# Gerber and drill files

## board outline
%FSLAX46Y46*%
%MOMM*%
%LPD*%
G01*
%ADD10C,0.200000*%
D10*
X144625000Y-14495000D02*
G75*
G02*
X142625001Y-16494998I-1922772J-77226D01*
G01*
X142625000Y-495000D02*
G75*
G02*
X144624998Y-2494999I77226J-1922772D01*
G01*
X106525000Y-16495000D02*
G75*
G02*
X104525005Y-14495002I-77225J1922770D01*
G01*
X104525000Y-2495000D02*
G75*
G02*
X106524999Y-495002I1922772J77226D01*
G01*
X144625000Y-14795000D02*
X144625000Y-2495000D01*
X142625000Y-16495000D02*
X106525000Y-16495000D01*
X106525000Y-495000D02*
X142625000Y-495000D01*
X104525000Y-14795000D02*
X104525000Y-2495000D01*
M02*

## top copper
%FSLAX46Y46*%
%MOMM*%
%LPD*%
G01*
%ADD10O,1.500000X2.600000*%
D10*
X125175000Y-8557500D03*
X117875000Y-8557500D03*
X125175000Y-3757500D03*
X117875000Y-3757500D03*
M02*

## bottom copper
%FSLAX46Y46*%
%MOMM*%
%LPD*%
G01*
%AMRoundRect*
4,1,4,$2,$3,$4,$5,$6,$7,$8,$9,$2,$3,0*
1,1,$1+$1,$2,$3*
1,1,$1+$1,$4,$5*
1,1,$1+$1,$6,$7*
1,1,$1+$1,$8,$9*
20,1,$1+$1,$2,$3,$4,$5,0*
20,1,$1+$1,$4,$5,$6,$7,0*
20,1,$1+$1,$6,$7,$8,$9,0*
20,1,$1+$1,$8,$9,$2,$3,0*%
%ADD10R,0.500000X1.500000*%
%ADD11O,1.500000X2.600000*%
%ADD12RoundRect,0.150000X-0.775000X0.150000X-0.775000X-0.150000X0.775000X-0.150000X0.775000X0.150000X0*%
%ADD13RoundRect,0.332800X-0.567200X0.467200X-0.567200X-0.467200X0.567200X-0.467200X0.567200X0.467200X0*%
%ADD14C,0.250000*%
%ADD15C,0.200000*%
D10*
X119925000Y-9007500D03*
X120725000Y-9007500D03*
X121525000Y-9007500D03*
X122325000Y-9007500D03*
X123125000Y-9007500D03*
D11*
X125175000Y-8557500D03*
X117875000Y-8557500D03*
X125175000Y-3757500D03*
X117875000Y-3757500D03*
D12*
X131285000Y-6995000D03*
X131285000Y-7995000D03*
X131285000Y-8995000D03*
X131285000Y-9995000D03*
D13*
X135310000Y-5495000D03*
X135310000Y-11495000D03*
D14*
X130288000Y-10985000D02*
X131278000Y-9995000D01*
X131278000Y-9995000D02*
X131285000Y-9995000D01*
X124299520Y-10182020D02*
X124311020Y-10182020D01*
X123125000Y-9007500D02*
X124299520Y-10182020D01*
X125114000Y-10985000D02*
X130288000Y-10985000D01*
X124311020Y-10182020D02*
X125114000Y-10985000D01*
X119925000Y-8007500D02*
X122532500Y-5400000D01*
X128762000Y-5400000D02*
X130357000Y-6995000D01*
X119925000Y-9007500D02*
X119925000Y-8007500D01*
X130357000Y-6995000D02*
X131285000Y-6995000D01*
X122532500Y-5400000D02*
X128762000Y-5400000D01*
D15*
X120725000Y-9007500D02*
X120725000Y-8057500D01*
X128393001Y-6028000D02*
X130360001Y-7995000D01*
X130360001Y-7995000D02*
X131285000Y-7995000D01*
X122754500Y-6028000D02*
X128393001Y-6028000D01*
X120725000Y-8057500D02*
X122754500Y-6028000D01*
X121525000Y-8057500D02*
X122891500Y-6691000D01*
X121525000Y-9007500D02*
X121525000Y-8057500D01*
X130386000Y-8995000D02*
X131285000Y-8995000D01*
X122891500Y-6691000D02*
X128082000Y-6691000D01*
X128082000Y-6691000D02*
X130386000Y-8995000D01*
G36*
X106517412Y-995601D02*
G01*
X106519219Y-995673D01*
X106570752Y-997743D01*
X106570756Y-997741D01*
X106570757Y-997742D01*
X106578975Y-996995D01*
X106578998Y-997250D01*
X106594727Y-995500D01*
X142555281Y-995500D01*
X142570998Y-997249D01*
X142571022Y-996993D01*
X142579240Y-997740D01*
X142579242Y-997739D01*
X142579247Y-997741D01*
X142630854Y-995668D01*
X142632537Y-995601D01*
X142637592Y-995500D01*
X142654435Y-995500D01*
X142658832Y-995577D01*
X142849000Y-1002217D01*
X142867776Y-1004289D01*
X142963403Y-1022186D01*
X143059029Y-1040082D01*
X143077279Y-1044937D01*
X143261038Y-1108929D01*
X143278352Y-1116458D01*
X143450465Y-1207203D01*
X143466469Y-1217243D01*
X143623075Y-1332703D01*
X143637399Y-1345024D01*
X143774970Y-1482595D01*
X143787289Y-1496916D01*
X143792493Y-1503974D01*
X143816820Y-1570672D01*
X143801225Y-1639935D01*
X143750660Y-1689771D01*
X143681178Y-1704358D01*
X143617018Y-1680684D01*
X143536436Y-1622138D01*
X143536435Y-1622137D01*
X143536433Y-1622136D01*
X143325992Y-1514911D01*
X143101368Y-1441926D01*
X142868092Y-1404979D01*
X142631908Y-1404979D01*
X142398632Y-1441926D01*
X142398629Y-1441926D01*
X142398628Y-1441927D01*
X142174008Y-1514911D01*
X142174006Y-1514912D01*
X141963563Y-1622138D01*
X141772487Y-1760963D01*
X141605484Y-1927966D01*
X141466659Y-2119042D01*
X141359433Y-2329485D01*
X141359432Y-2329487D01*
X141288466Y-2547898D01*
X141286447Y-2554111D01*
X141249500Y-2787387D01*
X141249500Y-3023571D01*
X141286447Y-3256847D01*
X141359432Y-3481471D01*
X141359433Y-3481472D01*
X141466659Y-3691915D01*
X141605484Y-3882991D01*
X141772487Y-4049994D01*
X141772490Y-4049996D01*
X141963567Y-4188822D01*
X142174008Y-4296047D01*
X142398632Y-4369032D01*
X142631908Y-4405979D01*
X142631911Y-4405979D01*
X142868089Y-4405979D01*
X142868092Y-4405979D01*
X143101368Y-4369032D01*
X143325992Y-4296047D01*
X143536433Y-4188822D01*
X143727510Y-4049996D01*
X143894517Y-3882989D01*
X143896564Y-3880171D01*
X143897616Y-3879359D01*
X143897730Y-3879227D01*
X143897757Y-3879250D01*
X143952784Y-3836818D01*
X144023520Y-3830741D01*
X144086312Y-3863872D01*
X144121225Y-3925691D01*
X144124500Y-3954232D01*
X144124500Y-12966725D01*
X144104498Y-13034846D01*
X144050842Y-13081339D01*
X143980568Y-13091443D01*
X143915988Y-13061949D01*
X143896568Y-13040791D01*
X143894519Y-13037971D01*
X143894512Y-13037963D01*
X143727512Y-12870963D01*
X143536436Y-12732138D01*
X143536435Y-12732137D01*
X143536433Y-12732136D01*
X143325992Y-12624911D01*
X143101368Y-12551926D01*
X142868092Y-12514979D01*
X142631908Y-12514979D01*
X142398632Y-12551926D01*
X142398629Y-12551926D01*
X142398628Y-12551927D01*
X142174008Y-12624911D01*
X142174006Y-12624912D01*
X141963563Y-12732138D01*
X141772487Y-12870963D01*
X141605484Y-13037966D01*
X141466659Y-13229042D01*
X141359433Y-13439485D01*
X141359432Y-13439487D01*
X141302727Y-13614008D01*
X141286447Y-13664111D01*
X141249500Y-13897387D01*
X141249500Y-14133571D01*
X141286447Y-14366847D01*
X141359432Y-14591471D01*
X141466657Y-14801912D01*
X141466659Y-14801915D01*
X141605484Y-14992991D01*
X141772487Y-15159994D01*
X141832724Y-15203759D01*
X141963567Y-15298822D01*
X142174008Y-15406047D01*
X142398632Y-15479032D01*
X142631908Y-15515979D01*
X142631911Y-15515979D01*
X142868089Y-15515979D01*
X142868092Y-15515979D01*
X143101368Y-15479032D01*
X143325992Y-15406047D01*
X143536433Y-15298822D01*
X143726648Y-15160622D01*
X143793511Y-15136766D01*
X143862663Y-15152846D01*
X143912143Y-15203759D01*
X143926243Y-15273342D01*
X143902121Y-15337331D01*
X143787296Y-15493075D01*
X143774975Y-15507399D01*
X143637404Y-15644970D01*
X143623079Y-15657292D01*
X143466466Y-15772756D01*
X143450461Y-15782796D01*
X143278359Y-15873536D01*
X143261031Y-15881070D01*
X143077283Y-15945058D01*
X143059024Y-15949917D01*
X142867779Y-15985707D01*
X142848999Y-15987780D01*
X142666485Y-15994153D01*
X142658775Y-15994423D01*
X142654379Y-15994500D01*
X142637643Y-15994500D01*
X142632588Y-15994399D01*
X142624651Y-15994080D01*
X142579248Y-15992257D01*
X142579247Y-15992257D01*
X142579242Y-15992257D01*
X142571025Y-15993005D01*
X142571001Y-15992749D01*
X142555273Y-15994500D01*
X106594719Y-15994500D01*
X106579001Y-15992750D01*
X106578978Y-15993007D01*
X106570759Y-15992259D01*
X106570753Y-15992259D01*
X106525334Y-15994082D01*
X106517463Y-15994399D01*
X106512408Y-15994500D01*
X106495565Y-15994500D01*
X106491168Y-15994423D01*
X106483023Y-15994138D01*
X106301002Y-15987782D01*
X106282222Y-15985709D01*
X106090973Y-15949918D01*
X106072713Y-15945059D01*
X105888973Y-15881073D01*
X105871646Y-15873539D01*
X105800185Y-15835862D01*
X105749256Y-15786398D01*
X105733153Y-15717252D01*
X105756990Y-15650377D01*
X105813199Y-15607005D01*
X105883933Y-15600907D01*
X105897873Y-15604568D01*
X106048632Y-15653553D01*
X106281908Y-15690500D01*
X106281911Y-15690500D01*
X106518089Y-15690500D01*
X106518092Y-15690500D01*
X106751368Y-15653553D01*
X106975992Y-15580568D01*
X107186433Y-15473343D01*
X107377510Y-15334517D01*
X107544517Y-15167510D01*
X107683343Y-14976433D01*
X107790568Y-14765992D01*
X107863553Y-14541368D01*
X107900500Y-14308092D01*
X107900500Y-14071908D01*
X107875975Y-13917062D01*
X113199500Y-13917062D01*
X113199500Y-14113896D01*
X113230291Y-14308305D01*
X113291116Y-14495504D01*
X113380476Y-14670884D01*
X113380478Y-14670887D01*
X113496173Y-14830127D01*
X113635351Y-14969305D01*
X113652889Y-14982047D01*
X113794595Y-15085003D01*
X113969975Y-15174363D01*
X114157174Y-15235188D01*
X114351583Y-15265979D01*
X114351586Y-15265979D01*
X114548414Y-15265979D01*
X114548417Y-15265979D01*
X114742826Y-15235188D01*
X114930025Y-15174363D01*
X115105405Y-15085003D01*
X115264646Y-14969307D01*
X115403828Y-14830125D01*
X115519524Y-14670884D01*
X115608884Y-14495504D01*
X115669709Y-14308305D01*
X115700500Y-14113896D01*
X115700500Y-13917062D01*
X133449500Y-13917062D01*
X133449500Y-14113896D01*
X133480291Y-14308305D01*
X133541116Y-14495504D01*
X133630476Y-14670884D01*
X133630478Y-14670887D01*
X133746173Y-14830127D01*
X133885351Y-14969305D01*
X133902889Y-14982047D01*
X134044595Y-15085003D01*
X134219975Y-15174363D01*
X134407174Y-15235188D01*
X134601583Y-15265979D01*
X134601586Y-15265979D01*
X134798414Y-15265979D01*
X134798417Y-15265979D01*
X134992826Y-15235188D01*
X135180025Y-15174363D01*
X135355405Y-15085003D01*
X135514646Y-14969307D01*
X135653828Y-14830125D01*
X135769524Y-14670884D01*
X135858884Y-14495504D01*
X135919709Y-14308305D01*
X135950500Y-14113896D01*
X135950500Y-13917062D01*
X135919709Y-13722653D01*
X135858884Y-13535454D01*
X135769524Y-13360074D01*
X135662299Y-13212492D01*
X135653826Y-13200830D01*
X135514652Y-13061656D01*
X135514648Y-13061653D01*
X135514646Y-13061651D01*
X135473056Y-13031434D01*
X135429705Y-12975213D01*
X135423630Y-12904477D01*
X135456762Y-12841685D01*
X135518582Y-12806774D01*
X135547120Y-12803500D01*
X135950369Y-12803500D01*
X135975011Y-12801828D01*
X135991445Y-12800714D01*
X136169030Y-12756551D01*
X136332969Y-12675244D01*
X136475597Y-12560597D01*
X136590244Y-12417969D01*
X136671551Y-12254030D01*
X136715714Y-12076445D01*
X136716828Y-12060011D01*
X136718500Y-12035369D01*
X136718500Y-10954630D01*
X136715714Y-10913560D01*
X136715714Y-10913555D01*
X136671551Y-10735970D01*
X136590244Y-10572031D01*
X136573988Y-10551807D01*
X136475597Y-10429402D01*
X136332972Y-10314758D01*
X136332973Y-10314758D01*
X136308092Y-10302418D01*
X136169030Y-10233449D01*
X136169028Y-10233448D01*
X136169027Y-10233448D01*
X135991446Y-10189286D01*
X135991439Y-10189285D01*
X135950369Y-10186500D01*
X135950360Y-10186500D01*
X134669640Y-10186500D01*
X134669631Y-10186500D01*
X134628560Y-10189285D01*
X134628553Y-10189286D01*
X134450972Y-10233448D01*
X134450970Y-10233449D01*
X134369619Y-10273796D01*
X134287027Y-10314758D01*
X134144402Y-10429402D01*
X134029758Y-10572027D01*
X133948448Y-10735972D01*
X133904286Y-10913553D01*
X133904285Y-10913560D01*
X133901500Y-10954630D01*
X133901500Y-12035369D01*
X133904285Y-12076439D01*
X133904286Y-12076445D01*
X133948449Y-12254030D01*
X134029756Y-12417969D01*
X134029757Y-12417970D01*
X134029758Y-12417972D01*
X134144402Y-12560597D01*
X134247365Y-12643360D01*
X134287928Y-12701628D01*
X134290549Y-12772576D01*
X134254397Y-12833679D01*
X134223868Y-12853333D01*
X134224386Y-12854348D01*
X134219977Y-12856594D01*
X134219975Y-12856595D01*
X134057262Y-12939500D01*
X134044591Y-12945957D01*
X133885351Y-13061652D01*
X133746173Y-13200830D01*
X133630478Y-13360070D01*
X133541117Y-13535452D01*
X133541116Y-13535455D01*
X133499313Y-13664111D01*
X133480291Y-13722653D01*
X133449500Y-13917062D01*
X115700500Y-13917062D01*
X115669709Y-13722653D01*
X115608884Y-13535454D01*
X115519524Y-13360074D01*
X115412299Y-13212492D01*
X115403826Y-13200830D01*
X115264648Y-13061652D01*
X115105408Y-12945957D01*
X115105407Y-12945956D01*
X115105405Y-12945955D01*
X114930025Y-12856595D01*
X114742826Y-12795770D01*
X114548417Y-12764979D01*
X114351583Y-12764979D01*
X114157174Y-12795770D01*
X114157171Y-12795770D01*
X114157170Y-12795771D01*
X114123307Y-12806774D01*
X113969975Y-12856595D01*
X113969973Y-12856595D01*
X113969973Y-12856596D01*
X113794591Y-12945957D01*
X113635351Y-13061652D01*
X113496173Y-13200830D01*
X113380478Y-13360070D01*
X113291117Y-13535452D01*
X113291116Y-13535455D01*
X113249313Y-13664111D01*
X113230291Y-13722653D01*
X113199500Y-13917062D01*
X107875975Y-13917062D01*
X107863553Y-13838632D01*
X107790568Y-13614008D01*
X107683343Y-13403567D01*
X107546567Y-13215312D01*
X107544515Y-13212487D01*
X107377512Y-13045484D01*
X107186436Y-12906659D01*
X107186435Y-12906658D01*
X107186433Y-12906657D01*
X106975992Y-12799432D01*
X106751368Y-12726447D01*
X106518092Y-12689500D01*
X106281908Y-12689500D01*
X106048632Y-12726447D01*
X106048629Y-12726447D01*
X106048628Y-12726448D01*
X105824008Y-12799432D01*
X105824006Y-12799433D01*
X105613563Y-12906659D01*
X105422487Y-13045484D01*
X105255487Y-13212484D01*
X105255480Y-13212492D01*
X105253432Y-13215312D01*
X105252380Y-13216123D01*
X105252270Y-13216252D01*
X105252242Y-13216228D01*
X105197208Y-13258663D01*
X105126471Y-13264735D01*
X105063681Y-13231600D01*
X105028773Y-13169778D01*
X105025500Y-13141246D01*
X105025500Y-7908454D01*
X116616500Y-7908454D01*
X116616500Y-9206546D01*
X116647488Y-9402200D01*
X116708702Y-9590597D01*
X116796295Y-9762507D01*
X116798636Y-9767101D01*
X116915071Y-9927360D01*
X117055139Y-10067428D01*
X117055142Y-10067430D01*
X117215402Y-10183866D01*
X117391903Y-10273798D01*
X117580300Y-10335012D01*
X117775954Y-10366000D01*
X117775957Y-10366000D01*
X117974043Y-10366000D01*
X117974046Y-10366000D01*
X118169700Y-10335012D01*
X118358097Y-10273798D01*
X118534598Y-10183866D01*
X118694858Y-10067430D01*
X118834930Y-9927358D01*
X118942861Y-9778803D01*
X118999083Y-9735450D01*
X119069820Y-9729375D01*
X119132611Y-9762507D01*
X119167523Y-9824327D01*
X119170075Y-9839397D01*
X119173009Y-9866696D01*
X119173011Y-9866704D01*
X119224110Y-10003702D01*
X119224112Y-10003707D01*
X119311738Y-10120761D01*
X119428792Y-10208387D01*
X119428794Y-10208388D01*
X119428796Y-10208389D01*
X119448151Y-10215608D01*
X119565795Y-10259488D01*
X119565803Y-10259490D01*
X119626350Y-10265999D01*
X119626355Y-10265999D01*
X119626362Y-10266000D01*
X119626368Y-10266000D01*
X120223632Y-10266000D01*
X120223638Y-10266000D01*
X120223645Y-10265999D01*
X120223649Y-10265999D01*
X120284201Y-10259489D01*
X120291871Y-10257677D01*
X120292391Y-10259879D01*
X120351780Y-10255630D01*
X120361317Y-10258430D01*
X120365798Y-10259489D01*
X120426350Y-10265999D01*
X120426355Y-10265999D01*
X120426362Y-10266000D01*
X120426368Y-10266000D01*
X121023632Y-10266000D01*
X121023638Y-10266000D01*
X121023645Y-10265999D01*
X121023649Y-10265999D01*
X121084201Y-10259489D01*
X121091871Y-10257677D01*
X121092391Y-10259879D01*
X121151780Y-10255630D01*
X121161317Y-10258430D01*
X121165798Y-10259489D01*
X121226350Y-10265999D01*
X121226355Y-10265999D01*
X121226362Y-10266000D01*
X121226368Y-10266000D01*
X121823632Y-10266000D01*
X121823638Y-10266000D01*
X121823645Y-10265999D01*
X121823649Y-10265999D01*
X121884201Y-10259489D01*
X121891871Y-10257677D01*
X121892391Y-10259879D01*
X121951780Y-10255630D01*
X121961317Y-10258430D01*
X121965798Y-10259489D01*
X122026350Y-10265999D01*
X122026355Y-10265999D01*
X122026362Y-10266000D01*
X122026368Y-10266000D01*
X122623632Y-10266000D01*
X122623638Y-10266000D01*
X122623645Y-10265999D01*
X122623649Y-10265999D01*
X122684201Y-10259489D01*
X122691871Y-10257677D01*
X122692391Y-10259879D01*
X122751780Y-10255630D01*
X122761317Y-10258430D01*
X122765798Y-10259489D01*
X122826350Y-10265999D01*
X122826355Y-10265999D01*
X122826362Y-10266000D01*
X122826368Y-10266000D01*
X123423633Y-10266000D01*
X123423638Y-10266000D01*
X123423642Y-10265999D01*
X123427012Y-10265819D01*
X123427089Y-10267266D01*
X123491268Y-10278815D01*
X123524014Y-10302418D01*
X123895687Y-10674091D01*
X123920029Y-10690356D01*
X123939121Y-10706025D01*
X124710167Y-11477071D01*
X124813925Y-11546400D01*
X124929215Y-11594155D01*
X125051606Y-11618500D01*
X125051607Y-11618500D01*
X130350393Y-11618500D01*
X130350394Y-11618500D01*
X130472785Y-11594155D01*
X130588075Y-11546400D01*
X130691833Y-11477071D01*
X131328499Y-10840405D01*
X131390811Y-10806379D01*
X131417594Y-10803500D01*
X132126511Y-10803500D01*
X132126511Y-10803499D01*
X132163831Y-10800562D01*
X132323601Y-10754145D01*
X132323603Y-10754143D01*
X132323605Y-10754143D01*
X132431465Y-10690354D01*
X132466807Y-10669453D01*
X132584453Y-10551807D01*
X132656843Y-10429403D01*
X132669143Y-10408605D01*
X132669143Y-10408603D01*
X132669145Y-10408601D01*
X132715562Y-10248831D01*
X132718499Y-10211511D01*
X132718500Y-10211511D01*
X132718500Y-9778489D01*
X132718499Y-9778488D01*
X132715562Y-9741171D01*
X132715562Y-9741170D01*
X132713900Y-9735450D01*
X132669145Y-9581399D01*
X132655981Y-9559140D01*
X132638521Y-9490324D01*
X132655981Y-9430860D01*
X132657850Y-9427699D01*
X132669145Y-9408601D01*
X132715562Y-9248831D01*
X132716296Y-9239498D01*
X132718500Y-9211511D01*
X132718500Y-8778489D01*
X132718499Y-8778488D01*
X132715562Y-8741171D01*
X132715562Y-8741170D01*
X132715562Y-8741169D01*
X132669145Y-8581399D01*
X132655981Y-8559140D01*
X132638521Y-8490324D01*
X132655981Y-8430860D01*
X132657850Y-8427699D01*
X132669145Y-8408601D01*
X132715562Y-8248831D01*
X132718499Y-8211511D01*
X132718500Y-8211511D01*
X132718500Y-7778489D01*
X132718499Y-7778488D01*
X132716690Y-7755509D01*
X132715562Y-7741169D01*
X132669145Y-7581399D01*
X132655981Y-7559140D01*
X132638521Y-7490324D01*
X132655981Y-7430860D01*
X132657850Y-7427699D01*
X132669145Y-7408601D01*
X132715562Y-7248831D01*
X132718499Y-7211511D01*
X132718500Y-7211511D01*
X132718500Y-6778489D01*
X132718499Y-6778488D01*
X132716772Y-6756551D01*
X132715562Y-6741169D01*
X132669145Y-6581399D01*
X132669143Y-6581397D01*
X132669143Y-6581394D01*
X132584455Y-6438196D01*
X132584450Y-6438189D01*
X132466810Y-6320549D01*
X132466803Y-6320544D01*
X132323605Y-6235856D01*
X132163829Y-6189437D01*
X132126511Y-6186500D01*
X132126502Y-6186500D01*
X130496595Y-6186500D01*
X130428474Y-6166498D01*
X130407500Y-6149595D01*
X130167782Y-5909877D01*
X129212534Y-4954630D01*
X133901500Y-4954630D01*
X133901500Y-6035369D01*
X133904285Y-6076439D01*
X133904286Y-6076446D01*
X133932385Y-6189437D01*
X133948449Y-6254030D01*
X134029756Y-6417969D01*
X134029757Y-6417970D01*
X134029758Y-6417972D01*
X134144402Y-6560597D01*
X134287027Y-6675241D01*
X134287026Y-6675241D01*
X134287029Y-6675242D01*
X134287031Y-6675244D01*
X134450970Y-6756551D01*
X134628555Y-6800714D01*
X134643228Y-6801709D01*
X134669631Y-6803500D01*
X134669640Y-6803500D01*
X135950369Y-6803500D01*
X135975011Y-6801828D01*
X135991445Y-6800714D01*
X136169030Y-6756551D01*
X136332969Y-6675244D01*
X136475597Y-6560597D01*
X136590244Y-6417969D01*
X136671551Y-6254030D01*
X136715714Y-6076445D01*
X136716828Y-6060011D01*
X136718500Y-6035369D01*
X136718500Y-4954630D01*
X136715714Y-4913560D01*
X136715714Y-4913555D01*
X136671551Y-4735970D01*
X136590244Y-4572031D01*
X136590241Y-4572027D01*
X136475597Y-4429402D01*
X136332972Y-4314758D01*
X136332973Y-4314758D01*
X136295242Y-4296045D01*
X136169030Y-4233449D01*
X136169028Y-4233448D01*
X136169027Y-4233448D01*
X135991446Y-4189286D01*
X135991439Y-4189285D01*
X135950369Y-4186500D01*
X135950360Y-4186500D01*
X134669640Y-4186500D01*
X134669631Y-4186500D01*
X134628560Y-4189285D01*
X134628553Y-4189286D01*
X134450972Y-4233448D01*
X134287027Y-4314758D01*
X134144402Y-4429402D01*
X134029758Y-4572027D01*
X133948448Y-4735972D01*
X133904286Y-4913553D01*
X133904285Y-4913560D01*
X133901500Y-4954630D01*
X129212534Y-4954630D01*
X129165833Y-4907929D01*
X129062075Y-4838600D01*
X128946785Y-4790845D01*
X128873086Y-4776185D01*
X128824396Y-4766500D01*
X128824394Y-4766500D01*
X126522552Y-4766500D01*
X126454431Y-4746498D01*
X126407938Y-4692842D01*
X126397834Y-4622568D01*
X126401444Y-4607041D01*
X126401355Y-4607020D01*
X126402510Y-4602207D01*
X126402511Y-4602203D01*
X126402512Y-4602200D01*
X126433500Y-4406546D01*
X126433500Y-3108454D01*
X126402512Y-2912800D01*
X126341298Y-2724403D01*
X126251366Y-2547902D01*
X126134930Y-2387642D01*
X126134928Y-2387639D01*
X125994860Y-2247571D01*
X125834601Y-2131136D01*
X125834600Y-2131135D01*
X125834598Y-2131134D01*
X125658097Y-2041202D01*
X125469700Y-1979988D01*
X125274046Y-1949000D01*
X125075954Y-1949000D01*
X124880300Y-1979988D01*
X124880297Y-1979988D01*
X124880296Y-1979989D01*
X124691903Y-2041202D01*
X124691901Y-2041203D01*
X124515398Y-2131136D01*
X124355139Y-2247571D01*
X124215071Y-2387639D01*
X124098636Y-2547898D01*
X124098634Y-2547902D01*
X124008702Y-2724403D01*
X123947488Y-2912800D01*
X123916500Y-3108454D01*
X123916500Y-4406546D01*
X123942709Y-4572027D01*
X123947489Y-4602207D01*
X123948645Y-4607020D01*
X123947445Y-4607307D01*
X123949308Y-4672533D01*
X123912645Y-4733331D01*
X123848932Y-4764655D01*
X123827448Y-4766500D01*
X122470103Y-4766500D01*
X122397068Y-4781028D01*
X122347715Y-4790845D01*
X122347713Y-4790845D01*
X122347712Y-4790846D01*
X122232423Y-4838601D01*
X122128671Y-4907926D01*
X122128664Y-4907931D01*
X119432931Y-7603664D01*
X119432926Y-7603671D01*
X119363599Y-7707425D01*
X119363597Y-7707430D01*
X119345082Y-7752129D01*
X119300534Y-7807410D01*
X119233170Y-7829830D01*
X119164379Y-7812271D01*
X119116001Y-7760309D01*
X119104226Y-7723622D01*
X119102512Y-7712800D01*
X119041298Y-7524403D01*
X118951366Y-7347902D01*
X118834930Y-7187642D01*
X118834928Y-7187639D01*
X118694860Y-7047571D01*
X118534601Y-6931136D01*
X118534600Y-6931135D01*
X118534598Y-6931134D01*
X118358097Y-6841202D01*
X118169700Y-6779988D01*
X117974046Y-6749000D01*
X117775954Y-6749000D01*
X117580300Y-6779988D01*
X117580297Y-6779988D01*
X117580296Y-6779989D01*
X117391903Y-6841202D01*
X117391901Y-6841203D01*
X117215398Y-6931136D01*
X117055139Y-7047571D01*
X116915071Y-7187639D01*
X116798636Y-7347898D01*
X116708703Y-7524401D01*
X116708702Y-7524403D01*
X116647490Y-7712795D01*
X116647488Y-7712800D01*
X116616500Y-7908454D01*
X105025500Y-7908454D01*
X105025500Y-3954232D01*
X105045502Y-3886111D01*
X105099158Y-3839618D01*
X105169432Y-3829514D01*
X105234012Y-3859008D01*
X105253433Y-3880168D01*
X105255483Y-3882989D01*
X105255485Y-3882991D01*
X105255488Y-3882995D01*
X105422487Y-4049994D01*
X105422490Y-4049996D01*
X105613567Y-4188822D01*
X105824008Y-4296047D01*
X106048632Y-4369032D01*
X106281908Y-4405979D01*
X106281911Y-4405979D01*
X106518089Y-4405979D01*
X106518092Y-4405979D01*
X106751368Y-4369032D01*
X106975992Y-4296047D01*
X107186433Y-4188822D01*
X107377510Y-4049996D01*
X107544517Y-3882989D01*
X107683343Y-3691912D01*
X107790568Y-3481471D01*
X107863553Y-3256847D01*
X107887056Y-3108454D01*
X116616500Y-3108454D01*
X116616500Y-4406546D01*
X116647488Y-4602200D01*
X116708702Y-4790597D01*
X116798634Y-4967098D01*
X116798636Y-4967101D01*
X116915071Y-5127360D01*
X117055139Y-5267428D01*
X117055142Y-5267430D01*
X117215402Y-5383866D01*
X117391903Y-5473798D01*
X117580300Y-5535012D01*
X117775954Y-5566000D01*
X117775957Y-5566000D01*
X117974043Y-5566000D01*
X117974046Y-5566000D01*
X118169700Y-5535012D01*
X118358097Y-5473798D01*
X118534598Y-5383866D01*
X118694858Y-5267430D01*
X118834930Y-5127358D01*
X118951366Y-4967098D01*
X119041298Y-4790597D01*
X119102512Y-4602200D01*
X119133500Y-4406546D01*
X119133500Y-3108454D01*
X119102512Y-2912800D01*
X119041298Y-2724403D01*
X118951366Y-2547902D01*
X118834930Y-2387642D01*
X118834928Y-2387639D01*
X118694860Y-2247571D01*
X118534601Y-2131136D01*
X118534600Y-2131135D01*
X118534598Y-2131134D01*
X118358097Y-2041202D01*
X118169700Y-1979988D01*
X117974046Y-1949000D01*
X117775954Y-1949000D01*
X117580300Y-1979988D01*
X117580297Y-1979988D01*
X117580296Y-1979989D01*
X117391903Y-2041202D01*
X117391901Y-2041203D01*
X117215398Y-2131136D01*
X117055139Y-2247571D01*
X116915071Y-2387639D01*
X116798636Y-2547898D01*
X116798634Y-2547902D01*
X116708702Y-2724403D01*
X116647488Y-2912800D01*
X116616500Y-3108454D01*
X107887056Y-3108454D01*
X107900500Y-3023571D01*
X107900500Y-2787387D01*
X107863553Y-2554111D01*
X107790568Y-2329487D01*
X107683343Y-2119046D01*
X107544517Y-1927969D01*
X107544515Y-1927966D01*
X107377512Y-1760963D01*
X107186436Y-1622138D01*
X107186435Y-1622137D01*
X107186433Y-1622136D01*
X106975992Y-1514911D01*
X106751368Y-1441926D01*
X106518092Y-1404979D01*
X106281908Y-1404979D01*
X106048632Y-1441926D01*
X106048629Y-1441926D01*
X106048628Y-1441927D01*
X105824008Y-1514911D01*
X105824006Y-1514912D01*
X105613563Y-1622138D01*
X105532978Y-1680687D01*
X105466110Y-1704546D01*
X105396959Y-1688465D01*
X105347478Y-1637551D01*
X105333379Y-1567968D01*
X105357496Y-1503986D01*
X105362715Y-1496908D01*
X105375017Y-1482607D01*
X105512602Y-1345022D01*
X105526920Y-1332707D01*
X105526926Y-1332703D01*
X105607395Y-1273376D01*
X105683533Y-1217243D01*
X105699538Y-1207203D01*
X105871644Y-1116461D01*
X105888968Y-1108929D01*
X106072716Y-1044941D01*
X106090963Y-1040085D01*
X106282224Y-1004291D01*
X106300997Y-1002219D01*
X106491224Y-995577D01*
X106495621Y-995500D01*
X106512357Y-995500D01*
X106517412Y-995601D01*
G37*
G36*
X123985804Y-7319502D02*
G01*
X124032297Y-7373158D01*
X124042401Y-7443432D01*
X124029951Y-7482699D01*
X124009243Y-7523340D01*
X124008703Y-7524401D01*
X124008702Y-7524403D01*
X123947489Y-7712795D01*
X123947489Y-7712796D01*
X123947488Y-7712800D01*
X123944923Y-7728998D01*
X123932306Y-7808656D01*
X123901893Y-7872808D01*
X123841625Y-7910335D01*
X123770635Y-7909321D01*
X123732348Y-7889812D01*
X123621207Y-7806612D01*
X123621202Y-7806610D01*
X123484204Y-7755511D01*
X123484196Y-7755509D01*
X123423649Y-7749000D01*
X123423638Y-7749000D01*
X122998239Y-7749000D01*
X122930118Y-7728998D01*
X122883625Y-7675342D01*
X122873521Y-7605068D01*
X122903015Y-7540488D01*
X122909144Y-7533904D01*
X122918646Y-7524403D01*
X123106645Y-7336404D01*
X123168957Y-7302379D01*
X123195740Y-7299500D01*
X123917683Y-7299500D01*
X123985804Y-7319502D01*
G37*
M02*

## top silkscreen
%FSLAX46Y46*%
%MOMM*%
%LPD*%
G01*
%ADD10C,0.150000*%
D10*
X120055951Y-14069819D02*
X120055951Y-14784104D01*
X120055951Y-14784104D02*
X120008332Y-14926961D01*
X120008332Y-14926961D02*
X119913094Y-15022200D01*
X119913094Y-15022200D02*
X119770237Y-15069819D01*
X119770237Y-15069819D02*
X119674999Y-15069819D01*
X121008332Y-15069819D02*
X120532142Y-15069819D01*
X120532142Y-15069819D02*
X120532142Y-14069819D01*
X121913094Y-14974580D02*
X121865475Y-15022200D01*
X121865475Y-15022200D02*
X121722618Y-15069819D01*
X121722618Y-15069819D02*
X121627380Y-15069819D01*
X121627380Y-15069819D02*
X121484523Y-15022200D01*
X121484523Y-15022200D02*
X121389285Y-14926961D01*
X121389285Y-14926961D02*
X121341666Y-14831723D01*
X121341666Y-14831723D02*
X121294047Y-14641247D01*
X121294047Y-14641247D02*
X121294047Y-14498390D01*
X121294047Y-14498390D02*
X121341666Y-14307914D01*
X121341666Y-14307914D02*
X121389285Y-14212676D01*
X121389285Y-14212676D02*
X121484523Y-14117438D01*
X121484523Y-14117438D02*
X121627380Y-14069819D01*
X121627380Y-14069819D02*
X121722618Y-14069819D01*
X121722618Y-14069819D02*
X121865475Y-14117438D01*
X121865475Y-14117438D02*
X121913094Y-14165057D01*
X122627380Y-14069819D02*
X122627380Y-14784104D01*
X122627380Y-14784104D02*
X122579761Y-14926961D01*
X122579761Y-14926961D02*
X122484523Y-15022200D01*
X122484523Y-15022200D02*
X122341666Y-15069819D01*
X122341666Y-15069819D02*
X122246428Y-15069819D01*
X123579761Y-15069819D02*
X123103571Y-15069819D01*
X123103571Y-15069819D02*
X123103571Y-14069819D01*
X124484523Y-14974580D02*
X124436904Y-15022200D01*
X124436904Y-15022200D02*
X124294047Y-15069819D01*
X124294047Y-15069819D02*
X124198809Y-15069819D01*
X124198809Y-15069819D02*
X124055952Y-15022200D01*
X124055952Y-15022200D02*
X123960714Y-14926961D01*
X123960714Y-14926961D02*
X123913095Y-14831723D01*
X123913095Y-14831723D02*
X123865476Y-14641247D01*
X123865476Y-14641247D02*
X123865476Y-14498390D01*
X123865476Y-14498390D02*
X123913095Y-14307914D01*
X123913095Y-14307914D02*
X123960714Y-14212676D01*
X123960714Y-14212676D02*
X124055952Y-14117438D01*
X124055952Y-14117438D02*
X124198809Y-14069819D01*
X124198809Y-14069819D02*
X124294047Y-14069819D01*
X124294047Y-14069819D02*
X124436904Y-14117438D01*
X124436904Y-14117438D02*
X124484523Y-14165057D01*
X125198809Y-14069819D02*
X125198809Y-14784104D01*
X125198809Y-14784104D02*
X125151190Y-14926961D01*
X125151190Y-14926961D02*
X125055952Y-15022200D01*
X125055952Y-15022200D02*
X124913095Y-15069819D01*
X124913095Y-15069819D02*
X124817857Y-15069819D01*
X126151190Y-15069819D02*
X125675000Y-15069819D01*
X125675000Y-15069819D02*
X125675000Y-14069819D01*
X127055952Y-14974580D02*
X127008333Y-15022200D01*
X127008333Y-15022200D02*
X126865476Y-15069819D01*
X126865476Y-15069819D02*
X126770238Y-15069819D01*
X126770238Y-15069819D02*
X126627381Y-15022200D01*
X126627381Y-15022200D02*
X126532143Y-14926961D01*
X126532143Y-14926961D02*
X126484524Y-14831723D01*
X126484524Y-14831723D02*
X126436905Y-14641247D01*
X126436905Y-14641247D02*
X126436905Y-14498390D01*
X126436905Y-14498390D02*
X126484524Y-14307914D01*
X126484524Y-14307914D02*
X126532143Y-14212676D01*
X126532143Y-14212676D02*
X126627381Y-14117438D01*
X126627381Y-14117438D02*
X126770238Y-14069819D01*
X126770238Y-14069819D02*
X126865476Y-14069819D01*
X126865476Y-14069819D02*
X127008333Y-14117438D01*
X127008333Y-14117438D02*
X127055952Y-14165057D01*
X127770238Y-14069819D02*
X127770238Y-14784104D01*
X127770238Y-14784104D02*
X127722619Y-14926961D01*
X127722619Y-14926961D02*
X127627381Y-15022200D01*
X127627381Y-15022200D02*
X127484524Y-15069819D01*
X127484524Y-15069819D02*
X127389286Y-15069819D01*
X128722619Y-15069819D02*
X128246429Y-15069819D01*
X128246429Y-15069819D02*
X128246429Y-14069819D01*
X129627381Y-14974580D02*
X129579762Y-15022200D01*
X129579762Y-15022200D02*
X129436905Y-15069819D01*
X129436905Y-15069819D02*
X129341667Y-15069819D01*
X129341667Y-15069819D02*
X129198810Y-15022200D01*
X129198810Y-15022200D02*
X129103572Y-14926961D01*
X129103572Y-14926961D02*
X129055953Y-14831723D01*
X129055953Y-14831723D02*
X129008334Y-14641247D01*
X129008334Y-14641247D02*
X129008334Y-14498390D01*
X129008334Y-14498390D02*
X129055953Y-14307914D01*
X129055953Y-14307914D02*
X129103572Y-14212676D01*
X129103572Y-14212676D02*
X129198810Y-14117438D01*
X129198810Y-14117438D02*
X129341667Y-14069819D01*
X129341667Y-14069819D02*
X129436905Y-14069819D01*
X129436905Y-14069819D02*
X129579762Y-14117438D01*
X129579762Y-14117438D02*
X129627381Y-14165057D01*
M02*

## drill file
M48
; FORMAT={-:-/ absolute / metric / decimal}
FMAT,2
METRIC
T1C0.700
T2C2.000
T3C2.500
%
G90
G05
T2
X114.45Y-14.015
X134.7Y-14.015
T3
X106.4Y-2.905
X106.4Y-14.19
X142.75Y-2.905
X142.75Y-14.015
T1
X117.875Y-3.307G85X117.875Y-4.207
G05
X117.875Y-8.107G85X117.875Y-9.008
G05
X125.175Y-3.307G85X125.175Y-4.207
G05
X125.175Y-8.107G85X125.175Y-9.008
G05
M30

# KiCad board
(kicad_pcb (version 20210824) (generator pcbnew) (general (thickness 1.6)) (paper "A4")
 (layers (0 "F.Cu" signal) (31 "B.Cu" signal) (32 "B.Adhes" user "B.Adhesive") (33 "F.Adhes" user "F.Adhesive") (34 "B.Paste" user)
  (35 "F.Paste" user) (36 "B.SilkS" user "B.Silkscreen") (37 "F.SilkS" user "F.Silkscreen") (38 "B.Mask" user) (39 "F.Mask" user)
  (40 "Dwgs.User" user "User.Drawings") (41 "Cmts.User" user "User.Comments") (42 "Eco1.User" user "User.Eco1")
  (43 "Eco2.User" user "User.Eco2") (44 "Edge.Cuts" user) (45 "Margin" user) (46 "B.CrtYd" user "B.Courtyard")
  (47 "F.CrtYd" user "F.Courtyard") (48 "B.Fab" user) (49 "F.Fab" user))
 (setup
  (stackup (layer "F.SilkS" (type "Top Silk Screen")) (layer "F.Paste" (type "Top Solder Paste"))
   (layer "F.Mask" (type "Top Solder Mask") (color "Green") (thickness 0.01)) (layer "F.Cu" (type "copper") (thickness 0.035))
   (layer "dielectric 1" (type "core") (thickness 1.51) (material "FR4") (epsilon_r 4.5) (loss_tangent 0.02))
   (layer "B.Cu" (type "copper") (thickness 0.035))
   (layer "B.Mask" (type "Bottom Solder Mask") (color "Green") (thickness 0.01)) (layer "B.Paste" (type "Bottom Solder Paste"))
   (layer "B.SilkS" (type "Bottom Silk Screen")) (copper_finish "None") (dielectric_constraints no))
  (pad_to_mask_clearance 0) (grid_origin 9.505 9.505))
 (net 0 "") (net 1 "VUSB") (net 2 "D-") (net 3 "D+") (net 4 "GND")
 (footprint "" (layer "F.Cu") (at 136.255 14.205)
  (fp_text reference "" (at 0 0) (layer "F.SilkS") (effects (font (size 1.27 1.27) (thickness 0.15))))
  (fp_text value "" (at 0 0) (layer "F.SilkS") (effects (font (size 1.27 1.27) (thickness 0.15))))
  (pad "" np_thru_hole circle (at -1.555 -0.189521) (size 2 2) (drill 2) (layers F&B.Cu *.Mask)))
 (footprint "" (layer "F.Cu") (at 94.555 1.535)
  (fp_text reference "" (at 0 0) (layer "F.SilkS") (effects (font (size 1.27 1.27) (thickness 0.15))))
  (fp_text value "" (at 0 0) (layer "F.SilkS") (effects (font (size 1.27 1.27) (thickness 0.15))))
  (pad "" np_thru_hole circle (at 11.845 1.370479) (size 2.5 2.5) (drill 2.5) (layers F&B.Cu *.Mask)))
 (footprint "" (layer "F.Cu") (at 147.015 3.065)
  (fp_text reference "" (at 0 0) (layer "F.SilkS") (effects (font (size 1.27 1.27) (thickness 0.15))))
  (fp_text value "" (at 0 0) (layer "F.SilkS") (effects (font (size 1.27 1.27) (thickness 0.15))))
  (pad "" np_thru_hole circle (at -4.265 -0.159521) (size 2.5 2.5) (drill 2.5) (layers F&B.Cu *.Mask)))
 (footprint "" (layer "F.Cu") (at 94.295 7.445633)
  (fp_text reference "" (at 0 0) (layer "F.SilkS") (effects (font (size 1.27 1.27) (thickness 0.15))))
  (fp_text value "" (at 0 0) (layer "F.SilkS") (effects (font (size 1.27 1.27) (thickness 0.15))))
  (pad "" np_thru_hole circle (at 12.105 6.744367) (size 2.5 2.5) (drill 2.5) (layers F&B.Cu *.Mask)))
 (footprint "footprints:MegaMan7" (layer "F.Cu") (at 109.650838 8.415023)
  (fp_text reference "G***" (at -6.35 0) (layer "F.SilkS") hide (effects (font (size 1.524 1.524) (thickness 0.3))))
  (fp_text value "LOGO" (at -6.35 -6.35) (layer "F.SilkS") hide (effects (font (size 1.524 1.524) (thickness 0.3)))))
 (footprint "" (layer "F.Cu") (at 112.225 13.965)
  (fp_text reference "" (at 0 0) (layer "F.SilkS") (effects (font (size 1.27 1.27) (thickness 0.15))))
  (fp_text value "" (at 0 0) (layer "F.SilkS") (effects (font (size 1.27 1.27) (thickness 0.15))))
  (pad "" np_thru_hole circle (at 2.225 0.050479) (size 2 2) (drill 2) (layers F&B.Cu *.Mask)))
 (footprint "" (layer "F.Cu") (at 130.75 14.19)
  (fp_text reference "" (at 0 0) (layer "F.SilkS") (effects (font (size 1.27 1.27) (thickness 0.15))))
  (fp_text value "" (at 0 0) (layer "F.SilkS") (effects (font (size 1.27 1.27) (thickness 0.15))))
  (pad "" np_thru_hole circle (at 12 -0.174521) (size 2.5 2.5) (drill 2.5) (layers F&B.Cu *.Mask)))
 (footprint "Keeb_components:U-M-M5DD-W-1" (layer "B.Cu") (at 121.525 3.7575 180)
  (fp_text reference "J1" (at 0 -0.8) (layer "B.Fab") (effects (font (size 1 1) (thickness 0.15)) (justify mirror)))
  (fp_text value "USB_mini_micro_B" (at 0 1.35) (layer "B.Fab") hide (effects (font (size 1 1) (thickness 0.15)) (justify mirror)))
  (pad "1" smd rect locked (at 1.6 -5.25) (size 0.5 1.5) (layers "B.Cu" "B.Paste" "B.Mask") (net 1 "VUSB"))
  (pad "2" smd rect locked (at 0.8 -5.25) (size 0.5 1.5) (layers "B.Cu" "B.Paste" "B.Mask") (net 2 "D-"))
  (pad "3" smd rect locked (at 0 -5.25) (size 0.5 1.5) (layers "B.Cu" "B.Paste" "B.Mask") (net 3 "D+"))
  (pad "4" smd rect locked (at -0.8 -5.25) (size 0.5 1.5) (layers "B.Cu" "B.Paste" "B.Mask"))
  (pad "5" smd rect locked (at -1.6 -5.25) (size 0.5 1.5) (layers "B.Cu" "B.Paste" "B.Mask") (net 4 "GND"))
  (pad "6" thru_hole oval locked (at -3.65 -4.8) (size 1.5 2.6) (drill oval 0.7 1.6) (layers *.Cu *.Mask))
  (pad "6" thru_hole oval locked (at 3.65 -4.8) (size 1.5 2.6) (drill oval 0.7 1.6) (layers *.Cu *.Mask))
  (pad "6" thru_hole oval locked (at -3.65 0) (size 1.5 2.6) (drill oval 0.7 1.6) (layers *.Cu *.Mask))
  (pad "6" thru_hole oval locked (at 3.65 0) (size 1.5 2.6) (drill oval 0.7 1.6) (layers *.Cu *.Mask)))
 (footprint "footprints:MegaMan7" (layer "B.Cu") (at 109.67284 8.39588 180)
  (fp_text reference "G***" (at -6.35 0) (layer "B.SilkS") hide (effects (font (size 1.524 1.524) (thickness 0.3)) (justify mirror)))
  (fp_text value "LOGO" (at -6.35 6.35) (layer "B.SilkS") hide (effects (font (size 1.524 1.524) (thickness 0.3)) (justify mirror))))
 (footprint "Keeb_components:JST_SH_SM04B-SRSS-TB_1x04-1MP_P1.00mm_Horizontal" (layer "B.Cu") (at 133.435 8.495 -90)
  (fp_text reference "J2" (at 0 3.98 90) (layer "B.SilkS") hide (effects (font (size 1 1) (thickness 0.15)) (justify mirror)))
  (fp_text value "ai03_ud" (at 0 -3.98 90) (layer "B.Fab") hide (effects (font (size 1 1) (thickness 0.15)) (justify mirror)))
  (pad "1" smd roundrect locked (at -1.5 2.15 270) (size 0.6 1.85) (layers "B.Cu" "B.Paste" "B.Mask") (roundrect_rratio 0.25) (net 1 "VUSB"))
  (pad "2" smd roundrect locked (at -0.5 2.15 270) (size 0.6 1.85) (layers "B.Cu" "B.Paste" "B.Mask") (roundrect_rratio 0.25) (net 2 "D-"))
  (pad "3" smd roundrect locked (at 0.5 2.15 270) (size 0.6 1.85) (layers "B.Cu" "B.Paste" "B.Mask") (roundrect_rratio 0.25) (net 3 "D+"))
  (pad "4" smd roundrect locked (at 1.5 2.15 270) (size 0.6 1.85) (layers "B.Cu" "B.Paste" "B.Mask") (roundrect_rratio 0.25) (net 4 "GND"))
  (pad "MP" smd roundrect locked (at -3 -1.875 270) (size 1.6 1.8) (layers "B.Cu" "B.Paste" "B.Mask") (roundrect_rratio 0.208))
  (pad "MP" smd roundrect locked (at 3 -1.875 270) (size 1.6 1.8) (layers "B.Cu" "B.Paste" "B.Mask") (roundrect_rratio 0.208)))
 (gr_arc (start 142.702228 14.572226) (end 144.625 14.495) (angle 94.6) (layer "Edge.Cuts") (width 0.2))
 (gr_arc (start 142.702226 2.417772) (end 142.625 0.495) (angle 94.6) (layer "Edge.Cuts") (width 0.2))
 (gr_arc (start 106.447775 14.57223) (end 106.525 16.495) (angle 94.6) (layer "Edge.Cuts") (width 0.2))
 (gr_arc (start 106.447772 2.417774) (end 104.525 2.495) (angle 94.6) (layer "Edge.Cuts") (width 0.2))
 (gr_line (start 144.625 14.795) (end 144.625 2.495) (layer "Edge.Cuts") (width 0.2))
 (gr_line (start 142.625 16.495) (end 106.525 16.495) (layer "Edge.Cuts") (width 0.2))
 (gr_line (start 106.525 0.495) (end 142.625 0.495) (layer "Edge.Cuts") (width 0.2))
 (gr_line (start 104.525 14.795) (end 104.525 2.495) (layer "Edge.Cuts") (width 0.2))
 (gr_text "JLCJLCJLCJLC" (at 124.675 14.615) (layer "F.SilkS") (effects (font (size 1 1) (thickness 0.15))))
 (segment (start 130.288 10.985) (end 131.278 9.995) (width 0.25) (layer "B.Cu") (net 4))
 (segment (start 131.278 9.995) (end 131.285 9.995) (width 0.25) (layer "B.Cu") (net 4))
 (segment (start 124.29952 10.18202) (end 124.31102 10.18202) (width 0.25) (layer "B.Cu") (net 4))
 (segment (start 123.125 9.0075) (end 124.29952 10.18202) (width 0.25) (layer "B.Cu") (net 4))
 (segment (start 125.114 10.985) (end 130.288 10.985) (width 0.25) (layer "B.Cu") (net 4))
 (segment (start 124.31102 10.18202) (end 125.114 10.985) (width 0.25) (layer "B.Cu") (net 4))
 (segment (start 119.925 8.0075) (end 122.5325 5.4) (width 0.25) (layer "B.Cu") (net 1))
 (segment (start 128.762 5.4) (end 130.357 6.995) (width 0.25) (layer "B.Cu") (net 1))
 (segment (start 119.925 9.0075) (end 119.925 8.0075) (width 0.25) (layer "B.Cu") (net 1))
 (segment (start 130.357 6.995) (end 131.285 6.995) (width 0.25) (layer "B.Cu") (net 1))
 (segment (start 122.5325 5.4) (end 128.762 5.4) (width 0.25) (layer "B.Cu") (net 1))
 (segment (start 120.725 9.0075) (end 120.725 8.0575) (width 0.2) (layer "B.Cu") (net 2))
 (segment (start 128.393001 6.028) (end 130.360001 7.995) (width 0.2) (layer "B.Cu") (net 2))
 (segment (start 130.360001 7.995) (end 131.285 7.995) (width 0.2) (layer "B.Cu") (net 2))
 (segment (start 122.7545 6.028) (end 128.393001 6.028) (width 0.2) (layer "B.Cu") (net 2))
 (segment (start 120.725 8.0575) (end 122.7545 6.028) (width 0.2) (layer "B.Cu") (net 2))
 (segment (start 121.525 8.0575) (end 122.8915 6.691) (width 0.2) (layer "B.Cu") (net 3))
 (segment (start 121.525 9.0075) (end 121.525 8.0575) (width 0.2) (layer "B.Cu") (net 3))
 (segment (start 130.386 8.995) (end 131.285 8.995) (width 0.2) (layer "B.Cu") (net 3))
 (segment (start 122.8915 6.691) (end 128.082 6.691) (width 0.2) (layer "B.Cu") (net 3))
 (segment (start 128.082 6.691) (end 130.386 8.995) (width 0.2) (layer "B.Cu") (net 3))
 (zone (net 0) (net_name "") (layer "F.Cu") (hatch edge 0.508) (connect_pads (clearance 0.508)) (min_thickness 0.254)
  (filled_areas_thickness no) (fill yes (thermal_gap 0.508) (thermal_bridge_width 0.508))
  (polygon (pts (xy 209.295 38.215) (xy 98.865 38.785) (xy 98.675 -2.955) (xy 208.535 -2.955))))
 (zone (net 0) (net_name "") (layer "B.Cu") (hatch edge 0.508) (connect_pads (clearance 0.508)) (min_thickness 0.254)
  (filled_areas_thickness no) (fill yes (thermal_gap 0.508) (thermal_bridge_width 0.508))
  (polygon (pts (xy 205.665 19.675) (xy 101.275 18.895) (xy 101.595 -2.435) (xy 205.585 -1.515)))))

